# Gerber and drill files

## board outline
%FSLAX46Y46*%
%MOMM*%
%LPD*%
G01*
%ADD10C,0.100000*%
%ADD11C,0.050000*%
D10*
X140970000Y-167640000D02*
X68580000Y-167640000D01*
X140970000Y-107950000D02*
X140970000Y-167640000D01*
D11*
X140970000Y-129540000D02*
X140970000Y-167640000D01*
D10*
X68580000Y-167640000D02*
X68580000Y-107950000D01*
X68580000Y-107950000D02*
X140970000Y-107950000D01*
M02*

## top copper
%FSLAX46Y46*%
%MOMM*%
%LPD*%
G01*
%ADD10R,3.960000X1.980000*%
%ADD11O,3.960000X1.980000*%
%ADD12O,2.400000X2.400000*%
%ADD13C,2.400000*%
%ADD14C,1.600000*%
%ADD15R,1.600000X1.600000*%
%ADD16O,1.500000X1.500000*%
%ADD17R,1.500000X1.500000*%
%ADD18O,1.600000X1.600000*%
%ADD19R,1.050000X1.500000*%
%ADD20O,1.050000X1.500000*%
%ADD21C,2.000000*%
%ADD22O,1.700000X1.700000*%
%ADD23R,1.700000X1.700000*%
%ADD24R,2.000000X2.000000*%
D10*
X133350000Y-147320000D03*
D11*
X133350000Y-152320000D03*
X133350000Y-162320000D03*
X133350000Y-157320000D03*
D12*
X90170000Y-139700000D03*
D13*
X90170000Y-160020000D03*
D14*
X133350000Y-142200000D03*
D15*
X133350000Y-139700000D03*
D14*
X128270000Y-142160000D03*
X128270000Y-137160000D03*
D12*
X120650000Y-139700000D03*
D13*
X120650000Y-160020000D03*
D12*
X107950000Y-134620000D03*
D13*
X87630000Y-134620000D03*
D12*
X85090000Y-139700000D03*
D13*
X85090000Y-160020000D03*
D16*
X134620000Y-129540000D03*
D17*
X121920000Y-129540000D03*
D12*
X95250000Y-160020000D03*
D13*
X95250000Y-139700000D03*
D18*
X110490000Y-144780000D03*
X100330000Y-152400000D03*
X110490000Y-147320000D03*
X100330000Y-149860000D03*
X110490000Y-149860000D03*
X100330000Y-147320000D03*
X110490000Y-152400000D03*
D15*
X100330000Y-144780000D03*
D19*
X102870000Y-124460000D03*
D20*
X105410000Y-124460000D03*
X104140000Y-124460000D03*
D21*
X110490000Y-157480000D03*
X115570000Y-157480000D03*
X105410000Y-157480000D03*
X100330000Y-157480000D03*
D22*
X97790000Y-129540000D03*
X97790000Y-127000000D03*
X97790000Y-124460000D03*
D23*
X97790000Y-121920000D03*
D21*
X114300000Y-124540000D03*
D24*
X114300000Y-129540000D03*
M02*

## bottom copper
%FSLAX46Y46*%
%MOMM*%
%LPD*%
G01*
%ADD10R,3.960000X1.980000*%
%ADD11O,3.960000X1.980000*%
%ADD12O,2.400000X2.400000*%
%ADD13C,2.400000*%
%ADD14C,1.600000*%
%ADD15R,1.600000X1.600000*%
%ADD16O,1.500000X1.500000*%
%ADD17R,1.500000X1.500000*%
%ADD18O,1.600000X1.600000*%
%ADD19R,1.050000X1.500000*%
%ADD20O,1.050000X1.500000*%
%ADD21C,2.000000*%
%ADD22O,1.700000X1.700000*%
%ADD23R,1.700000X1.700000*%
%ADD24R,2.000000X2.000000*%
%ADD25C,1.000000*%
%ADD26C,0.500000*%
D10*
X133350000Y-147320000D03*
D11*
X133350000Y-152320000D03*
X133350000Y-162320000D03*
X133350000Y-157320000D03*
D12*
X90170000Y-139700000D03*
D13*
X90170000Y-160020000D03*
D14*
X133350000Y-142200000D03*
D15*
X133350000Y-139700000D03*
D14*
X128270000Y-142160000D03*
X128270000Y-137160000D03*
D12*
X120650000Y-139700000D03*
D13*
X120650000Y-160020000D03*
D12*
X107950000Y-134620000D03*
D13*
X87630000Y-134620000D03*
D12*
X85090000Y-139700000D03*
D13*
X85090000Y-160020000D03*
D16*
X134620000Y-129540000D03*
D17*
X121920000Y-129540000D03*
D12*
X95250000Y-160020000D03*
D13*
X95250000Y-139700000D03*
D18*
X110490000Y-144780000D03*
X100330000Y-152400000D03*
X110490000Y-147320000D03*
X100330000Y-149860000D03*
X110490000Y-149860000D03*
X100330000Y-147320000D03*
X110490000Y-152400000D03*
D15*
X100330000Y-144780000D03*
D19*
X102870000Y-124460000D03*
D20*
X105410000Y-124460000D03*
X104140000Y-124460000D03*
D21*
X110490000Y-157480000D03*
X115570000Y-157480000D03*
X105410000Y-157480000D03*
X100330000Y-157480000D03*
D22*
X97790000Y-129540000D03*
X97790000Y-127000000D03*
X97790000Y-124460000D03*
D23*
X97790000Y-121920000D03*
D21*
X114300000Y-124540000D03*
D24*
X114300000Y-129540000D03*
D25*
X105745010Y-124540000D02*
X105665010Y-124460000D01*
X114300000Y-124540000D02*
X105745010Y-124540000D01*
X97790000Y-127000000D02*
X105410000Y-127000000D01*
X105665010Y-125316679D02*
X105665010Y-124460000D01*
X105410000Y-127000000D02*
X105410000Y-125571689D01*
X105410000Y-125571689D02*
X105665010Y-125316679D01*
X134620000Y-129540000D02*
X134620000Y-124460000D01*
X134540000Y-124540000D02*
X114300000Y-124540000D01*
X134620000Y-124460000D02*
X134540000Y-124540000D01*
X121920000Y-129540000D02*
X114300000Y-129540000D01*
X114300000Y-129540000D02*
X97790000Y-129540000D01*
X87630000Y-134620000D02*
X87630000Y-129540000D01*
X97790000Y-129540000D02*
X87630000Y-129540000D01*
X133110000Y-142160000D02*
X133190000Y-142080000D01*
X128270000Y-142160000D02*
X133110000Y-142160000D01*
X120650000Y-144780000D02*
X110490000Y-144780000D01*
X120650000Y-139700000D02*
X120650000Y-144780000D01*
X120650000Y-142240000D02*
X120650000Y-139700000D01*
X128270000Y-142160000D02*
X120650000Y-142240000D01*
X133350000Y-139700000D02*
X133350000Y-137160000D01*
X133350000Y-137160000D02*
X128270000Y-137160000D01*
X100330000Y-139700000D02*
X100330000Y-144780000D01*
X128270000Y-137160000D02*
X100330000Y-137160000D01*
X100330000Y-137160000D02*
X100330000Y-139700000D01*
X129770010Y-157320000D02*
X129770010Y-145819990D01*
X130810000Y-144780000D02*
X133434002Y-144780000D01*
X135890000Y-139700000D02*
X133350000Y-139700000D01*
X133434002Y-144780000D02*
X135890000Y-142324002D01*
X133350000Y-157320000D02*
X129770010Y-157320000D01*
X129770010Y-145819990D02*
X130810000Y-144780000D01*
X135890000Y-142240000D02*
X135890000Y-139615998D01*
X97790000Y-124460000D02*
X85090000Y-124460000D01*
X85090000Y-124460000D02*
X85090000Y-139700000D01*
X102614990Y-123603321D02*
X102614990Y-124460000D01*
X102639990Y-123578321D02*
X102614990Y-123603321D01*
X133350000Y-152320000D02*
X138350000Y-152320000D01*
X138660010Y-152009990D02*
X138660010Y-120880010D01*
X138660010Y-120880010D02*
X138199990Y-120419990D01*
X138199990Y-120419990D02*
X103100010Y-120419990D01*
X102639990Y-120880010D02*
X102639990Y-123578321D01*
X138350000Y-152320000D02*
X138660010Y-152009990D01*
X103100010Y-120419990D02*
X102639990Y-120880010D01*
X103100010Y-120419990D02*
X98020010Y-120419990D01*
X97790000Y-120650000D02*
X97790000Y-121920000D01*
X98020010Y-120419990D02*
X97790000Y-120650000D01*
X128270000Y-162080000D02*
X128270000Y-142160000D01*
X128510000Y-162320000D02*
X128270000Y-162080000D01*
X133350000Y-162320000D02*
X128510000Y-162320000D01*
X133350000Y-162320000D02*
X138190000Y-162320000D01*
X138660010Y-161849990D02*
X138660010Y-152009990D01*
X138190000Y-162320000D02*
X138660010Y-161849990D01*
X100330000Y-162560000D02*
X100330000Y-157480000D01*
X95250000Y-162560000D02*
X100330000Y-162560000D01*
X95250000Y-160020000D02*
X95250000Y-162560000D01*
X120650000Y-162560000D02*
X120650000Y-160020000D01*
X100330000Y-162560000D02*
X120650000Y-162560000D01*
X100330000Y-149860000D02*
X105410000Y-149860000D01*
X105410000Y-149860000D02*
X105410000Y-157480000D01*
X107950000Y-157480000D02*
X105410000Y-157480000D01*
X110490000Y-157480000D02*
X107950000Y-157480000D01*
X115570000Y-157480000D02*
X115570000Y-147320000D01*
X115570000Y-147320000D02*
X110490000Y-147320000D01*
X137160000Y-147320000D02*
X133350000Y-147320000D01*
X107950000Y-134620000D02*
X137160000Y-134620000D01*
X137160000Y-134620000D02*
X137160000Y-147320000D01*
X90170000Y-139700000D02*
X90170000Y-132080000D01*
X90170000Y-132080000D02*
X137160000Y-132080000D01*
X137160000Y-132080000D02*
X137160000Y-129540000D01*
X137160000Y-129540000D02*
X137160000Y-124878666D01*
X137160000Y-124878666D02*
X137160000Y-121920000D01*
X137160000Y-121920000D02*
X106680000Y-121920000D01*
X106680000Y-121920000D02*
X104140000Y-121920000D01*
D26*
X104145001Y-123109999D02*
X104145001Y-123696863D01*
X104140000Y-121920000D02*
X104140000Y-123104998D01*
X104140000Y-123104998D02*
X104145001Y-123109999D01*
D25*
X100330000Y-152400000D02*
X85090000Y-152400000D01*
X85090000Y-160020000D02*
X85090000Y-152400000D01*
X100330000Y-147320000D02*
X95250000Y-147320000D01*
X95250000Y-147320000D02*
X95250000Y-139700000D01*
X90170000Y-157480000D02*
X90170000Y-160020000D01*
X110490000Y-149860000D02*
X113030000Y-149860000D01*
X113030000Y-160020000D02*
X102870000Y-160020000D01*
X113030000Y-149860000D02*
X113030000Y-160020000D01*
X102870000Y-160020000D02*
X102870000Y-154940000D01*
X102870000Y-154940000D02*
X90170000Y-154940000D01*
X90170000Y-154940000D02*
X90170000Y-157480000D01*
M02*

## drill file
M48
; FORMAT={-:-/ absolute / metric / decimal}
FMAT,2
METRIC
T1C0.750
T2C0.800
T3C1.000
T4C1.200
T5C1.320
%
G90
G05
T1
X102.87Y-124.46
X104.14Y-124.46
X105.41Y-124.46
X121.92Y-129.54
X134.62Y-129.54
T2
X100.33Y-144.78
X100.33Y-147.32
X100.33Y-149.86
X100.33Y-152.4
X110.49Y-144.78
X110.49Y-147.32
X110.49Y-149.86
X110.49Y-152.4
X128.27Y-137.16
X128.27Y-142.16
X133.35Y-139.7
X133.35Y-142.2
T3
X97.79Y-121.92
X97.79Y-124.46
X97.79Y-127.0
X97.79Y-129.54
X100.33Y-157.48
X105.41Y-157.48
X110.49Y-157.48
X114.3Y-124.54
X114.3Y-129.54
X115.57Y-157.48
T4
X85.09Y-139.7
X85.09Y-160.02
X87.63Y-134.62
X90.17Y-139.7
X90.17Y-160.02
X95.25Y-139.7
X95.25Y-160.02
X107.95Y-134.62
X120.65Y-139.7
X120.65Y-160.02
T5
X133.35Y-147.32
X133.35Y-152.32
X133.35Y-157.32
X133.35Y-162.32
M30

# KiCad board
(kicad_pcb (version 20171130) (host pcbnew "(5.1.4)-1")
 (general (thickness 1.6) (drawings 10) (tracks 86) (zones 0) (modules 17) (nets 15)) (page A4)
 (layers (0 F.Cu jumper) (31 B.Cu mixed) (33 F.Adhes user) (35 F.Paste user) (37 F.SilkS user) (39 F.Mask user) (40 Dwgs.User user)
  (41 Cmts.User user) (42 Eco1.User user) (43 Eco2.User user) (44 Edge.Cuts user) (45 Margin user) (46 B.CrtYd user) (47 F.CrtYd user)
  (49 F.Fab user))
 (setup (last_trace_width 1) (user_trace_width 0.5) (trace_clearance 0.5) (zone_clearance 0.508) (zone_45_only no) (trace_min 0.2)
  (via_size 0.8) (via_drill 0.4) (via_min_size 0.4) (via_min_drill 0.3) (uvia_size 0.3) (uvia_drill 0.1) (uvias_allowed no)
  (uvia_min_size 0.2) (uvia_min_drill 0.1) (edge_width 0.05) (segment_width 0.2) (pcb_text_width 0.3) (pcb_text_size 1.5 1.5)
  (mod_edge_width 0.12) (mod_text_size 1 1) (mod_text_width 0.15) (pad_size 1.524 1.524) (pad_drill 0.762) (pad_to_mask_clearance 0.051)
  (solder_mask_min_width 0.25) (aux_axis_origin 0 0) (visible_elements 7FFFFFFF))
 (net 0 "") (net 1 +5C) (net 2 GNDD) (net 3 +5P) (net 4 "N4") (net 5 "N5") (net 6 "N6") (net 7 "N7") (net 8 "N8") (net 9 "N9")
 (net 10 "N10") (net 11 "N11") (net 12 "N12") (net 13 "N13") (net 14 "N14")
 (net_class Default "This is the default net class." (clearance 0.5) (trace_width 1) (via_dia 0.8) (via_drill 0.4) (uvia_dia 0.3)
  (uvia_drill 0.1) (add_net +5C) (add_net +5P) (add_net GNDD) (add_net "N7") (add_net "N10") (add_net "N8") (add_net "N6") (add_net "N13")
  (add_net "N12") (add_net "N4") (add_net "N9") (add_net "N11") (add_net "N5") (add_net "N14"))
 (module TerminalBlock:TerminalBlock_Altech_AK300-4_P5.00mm (layer F.Cu) (at 133.35 147.32 270)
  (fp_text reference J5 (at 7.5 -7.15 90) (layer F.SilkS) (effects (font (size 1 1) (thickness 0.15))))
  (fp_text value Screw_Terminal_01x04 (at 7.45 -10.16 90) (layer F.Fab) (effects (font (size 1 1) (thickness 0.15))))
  (pad 1 thru_hole rect (at 0 0 270) (size 1.98 3.96) (drill 1.32) (layers *.Cu *.Mask) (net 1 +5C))
  (pad 2 thru_hole oval (at 5 0 270) (size 1.98 3.96) (drill 1.32) (layers *.Cu *.Mask) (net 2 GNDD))
  (pad 4 thru_hole oval (at 15 0 270) (size 1.98 3.96) (drill 1.32) (layers *.Cu *.Mask) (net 2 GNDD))
  (pad 3 thru_hole oval (at 10 0 270) (size 1.98 3.96) (drill 1.32) (layers *.Cu *.Mask) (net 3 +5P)))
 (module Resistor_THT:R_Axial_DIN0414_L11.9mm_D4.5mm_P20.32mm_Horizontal (layer F.Cu) (at 90.17 160.02 90)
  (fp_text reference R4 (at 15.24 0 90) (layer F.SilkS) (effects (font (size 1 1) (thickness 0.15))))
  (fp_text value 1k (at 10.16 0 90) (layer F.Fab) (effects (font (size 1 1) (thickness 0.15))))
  (pad 2 thru_hole oval (at 20.32 0 90) (size 2.4 2.4) (drill 1.2) (layers *.Cu *.Mask) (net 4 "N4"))
  (pad 1 thru_hole circle (at 0 0 90) (size 2.4 2.4) (drill 1.2) (layers *.Cu *.Mask) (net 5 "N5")))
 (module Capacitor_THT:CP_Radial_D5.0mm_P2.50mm (layer F.Cu) (at 133.35 139.7 270)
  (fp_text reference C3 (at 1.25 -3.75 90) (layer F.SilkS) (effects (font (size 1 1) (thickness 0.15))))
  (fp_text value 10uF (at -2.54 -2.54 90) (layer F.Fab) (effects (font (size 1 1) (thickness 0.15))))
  (pad 2 thru_hole circle (at 2.5 0 270) (size 1.6 1.6) (drill 0.8) (layers *.Cu *.Mask) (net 2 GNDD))
  (pad 1 thru_hole rect (at 0 0 270) (size 1.6 1.6) (drill 0.8) (layers *.Cu *.Mask) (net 3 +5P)))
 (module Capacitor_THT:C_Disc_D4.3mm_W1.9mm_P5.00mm (layer F.Cu) (at 128.27 137.16 270)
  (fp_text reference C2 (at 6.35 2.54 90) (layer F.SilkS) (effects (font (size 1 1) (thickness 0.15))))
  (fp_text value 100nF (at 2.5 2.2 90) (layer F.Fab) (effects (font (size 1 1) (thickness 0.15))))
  (pad 2 thru_hole circle (at 5 0 270) (size 1.6 1.6) (drill 0.8) (layers *.Cu *.Mask) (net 2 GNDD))
  (pad 1 thru_hole circle (at 0 0 270) (size 1.6 1.6) (drill 0.8) (layers *.Cu *.Mask) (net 3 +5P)))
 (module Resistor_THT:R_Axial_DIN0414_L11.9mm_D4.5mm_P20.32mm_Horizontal (layer F.Cu) (at 120.65 160.02 90)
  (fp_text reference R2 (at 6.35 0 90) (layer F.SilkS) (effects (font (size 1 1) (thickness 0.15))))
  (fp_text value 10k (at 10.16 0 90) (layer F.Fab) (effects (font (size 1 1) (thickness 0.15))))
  (pad 2 thru_hole oval (at 20.32 0 90) (size 2.4 2.4) (drill 1.2) (layers *.Cu *.Mask) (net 2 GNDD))
  (pad 1 thru_hole circle (at 0 0 90) (size 2.4 2.4) (drill 1.2) (layers *.Cu *.Mask) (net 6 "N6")))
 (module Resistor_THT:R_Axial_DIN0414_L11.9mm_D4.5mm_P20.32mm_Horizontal (layer F.Cu) (at 87.63 134.62)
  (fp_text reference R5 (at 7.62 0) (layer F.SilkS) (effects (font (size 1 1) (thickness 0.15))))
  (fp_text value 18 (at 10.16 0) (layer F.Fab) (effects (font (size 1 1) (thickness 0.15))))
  (pad 2 thru_hole oval (at 20.32 0) (size 2.4 2.4) (drill 1.2) (layers *.Cu *.Mask) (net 1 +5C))
  (pad 1 thru_hole circle (at 0 0) (size 2.4 2.4) (drill 1.2) (layers *.Cu *.Mask) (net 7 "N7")))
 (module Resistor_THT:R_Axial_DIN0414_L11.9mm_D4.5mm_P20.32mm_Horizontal (layer F.Cu) (at 85.09 160.02 90)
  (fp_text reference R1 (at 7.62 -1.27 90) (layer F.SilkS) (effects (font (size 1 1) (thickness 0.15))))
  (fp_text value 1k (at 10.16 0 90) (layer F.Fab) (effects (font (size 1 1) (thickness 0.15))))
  (pad 2 thru_hole oval (at 20.32 0 90) (size 2.4 2.4) (drill 1.2) (layers *.Cu *.Mask) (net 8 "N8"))
  (pad 1 thru_hole circle (at 0 0 90) (size 2.4 2.4) (drill 1.2) (layers *.Cu *.Mask) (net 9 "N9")))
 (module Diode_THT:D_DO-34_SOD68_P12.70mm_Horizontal (layer F.Cu) (at 121.92 129.54)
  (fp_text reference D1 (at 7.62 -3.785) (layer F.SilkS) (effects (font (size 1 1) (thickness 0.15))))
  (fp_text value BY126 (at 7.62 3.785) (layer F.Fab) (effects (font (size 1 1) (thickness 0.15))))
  (pad 2 thru_hole oval (at 12.7 0) (size 1.5 1.5) (drill 0.75) (layers *.Cu *.Mask) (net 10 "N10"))
  (pad 1 thru_hole rect (at 0 0) (size 1.5 1.5) (drill 0.75) (layers *.Cu *.Mask) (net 7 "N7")))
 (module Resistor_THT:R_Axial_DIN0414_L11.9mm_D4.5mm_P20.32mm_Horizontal (layer F.Cu) (at 95.25 139.7 270)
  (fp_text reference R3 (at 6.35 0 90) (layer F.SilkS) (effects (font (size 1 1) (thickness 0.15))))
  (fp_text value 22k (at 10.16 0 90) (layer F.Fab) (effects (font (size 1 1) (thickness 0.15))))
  (pad 2 thru_hole oval (at 20.32 0 270) (size 2.4 2.4) (drill 1.2) (layers *.Cu *.Mask) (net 6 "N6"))
  (pad 1 thru_hole circle (at 0 0 270) (size 2.4 2.4) (drill 1.2) (layers *.Cu *.Mask) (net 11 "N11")))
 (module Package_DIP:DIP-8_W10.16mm (layer F.Cu) (at 100.33 144.78)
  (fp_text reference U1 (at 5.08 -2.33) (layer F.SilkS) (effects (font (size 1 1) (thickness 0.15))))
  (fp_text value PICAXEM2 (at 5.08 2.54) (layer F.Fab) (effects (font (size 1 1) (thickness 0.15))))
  (pad 8 thru_hole oval (at 10.16 0) (size 1.6 1.6) (drill 0.8) (layers *.Cu *.Mask) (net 2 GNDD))
  (pad 4 thru_hole oval (at 0 7.62) (size 1.6 1.6) (drill 0.8) (layers *.Cu *.Mask) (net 9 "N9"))
  (pad 7 thru_hole oval (at 10.16 2.54) (size 1.6 1.6) (drill 0.8) (layers *.Cu *.Mask) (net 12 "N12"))
  (pad 3 thru_hole oval (at 0 5.08) (size 1.6 1.6) (drill 0.8) (layers *.Cu *.Mask) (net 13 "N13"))
  (pad 6 thru_hole oval (at 10.16 5.08) (size 1.6 1.6) (drill 0.8) (layers *.Cu *.Mask) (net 5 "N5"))
  (pad 2 thru_hole oval (at 0 2.54) (size 1.6 1.6) (drill 0.8) (layers *.Cu *.Mask) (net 11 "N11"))
  (pad 5 thru_hole oval (at 10.16 7.62) (size 1.6 1.6) (drill 0.8) (layers *.Cu *.Mask) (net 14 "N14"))
  (pad 1 thru_hole rect (at 0 0) (size 1.6 1.6) (drill 0.8) (layers *.Cu *.Mask) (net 3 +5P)))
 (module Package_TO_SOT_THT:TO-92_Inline (layer F.Cu) (at 102.87 124.46)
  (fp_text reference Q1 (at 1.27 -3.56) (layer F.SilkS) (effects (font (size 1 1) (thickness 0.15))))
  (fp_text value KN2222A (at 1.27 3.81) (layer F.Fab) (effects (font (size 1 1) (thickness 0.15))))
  (pad 1 thru_hole rect (at 0 0) (size 1.05 1.5) (drill 0.75) (layers *.Cu *.Mask) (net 2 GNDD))
  (pad 3 thru_hole oval (at 2.54 0) (size 1.05 1.5) (drill 0.75) (layers *.Cu *.Mask) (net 10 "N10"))
  (pad 2 thru_hole oval (at 1.27 0) (size 1.05 1.5) (drill 0.75) (layers *.Cu *.Mask) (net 4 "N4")))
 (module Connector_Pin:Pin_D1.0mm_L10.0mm (layer F.Cu) (at 110.49 157.48)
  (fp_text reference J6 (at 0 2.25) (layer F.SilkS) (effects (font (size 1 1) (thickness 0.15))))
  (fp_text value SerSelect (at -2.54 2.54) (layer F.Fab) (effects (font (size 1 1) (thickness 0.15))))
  (pad 1 thru_hole circle (at 0 0) (size 2 2) (drill 1) (layers *.Cu *.Mask) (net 13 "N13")))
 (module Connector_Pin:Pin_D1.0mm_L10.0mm (layer F.Cu) (at 115.57 157.48)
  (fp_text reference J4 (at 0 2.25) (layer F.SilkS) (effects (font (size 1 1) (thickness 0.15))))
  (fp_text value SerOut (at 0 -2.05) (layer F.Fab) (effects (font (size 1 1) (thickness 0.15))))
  (pad 1 thru_hole circle (at 0 0) (size 2 2) (drill 1) (layers *.Cu *.Mask) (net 12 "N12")))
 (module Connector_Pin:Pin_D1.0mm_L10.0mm (layer F.Cu) (at 105.41 157.48)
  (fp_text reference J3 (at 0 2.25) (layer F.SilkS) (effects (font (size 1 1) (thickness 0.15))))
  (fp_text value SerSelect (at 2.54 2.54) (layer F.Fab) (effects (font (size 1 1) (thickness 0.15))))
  (pad 1 thru_hole circle (at 0 0) (size 2 2) (drill 1) (layers *.Cu *.Mask) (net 13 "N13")))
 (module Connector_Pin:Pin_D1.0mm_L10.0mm (layer F.Cu) (at 100.33 157.48)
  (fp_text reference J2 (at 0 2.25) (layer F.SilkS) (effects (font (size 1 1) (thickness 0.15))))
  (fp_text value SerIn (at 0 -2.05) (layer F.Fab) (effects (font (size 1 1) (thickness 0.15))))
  (pad 1 thru_hole circle (at 0 0) (size 2 2) (drill 1) (layers *.Cu *.Mask) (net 6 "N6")))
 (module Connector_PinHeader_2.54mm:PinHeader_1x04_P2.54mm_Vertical (layer F.Cu) (at 97.79 121.92)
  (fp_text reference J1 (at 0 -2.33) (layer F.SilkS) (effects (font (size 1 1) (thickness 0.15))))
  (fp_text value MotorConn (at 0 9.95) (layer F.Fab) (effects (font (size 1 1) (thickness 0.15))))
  (pad 4 thru_hole oval (at 0 7.62) (size 1.7 1.7) (drill 1) (layers *.Cu *.Mask) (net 7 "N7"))
  (pad 3 thru_hole oval (at 0 5.08) (size 1.7 1.7) (drill 1) (layers *.Cu *.Mask) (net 10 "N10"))
  (pad 2 thru_hole oval (at 0 2.54) (size 1.7 1.7) (drill 1) (layers *.Cu *.Mask) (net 8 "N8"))
  (pad 1 thru_hole rect (at 0 0) (size 1.7 1.7) (drill 1) (layers *.Cu *.Mask) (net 2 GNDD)))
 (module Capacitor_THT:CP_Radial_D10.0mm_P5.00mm (layer F.Cu) (at 114.3 129.54 90)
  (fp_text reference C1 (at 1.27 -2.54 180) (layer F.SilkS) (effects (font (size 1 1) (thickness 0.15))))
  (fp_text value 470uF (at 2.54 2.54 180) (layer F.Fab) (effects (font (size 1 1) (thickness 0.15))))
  (pad 2 thru_hole circle (at 5 0 90) (size 2 2) (drill 1) (layers *.Cu *.Mask) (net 10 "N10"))
  (pad 1 thru_hole rect (at 0 0 90) (size 2 2) (drill 1) (layers *.Cu *.Mask) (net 7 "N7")))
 (gr_line (start 140.97 167.64) (end 68.58 167.64) (layer Edge.Cuts) (width 0.1))
 (gr_line (start 140.97 107.95) (end 140.97 167.64) (layer Edge.Cuts) (width 0.1))
 (gr_line (start 140.97 129.54) (end 140.97 167.64) (layer Edge.Cuts) (width 0.05))
 (gr_line (start 68.58 167.64) (end 68.58 107.95) (layer Edge.Cuts) (width 0.1))
 (gr_line (start 68.58 107.95) (end 140.97 107.95) (layer Edge.Cuts) (width 0.1))
 (segment (start 105.74501 124.54) (end 105.66501 124.46) (width 1) (layer B.Cu) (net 10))
 (segment (start 114.3 124.54) (end 105.74501 124.54) (width 1) (layer B.Cu) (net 10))
 (segment (start 97.79 127) (end 105.41 127) (width 1) (layer B.Cu) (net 10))
 (segment (start 105.66501 125.316679) (end 105.66501 124.46) (width 1) (layer B.Cu) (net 10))
 (segment (start 105.41 127) (end 105.41 125.571689) (width 1) (layer B.Cu) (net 10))
 (segment (start 105.41 125.571689) (end 105.66501 125.316679) (width 1) (layer B.Cu) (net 10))
 (segment (start 134.62 129.54) (end 134.62 124.46) (width 1) (layer B.Cu) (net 10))
 (segment (start 134.54 124.54) (end 114.3 124.54) (width 1) (layer B.Cu) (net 10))
 (segment (start 134.62 124.46) (end 134.54 124.54) (width 1) (layer B.Cu) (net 10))
 (segment (start 121.92 129.54) (end 114.3 129.54) (width 1) (layer B.Cu) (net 7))
 (segment (start 114.3 129.54) (end 97.79 129.54) (width 1) (layer B.Cu) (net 7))
 (segment (start 87.63 134.62) (end 87.63 129.54) (width 1) (layer B.Cu) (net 7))
 (segment (start 97.79 129.54) (end 87.63 129.54) (width 1) (layer B.Cu) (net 7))
 (segment (start 133.11 142.16) (end 133.19 142.08) (width 1) (layer B.Cu) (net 2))
 (segment (start 128.27 142.16) (end 133.11 142.16) (width 1) (layer B.Cu) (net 2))
 (segment (start 120.65 144.78) (end 110.49 144.78) (width 1) (layer B.Cu) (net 2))
 (segment (start 120.65 139.7) (end 120.65 144.78) (width 1) (layer B.Cu) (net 2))
 (segment (start 120.65 142.24) (end 120.65 139.7) (width 1) (layer B.Cu) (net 2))
 (segment (start 128.27 142.16) (end 120.65 142.24) (width 1) (layer B.Cu) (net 2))
 (segment (start 133.35 139.7) (end 133.35 137.16) (width 1) (layer B.Cu) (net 3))
 (segment (start 133.35 137.16) (end 128.27 137.16) (width 1) (layer B.Cu) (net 3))
 (segment (start 100.33 139.7) (end 100.33 144.78) (width 1) (layer B.Cu) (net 3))
 (segment (start 128.27 137.16) (end 100.33 137.16) (width 1) (layer B.Cu) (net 3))
 (segment (start 100.33 137.16) (end 100.33 139.7) (width 1) (layer B.Cu) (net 3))
 (segment (start 129.77001 157.32) (end 129.77001 145.81999) (width 1) (layer B.Cu) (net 3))
 (segment (start 130.81 144.78) (end 133.434002 144.78) (width 1) (layer B.Cu) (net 3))
 (segment (start 135.89 139.7) (end 133.35 139.7) (width 1) (layer B.Cu) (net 3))
 (segment (start 133.434002 144.78) (end 135.89 142.324002) (width 1) (layer B.Cu) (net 3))
 (segment (start 133.35 157.32) (end 129.77001 157.32) (width 1) (layer B.Cu) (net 3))
 (segment (start 129.77001 145.81999) (end 130.81 144.78) (width 1) (layer B.Cu) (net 3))
 (segment (start 135.89 142.24) (end 135.89 139.615998) (width 1) (layer B.Cu) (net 3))
 (segment (start 97.79 124.46) (end 85.09 124.46) (width 1) (layer B.Cu) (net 8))
 (segment (start 85.09 124.46) (end 85.09 139.7) (width 1) (layer B.Cu) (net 8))
 (segment (start 102.61499 123.603321) (end 102.61499 124.46) (width 1) (layer B.Cu) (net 2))
 (segment (start 102.63999 123.578321) (end 102.61499 123.603321) (width 1) (layer B.Cu) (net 2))
 (segment (start 133.35 152.32) (end 138.35 152.32) (width 1) (layer B.Cu) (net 2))
 (segment (start 138.66001 152.00999) (end 138.66001 120.88001) (width 1) (layer B.Cu) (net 2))
 (segment (start 138.66001 120.88001) (end 138.19999 120.41999) (width 1) (layer B.Cu) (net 2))
 (segment (start 138.19999 120.41999) (end 103.10001 120.41999) (width 1) (layer B.Cu) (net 2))
 (segment (start 102.63999 120.88001) (end 102.63999 123.578321) (width 1) (layer B.Cu) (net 2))
 (segment (start 138.35 152.32) (end 138.66001 152.00999) (width 1) (layer B.Cu) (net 2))
 (segment (start 103.10001 120.41999) (end 102.63999 120.88001) (width 1) (layer B.Cu) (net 2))
 (segment (start 103.10001 120.41999) (end 98.02001 120.41999) (width 1) (layer B.Cu) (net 2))
 (segment (start 97.79 120.65) (end 97.79 121.92) (width 1) (layer B.Cu) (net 2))
 (segment (start 98.02001 120.41999) (end 97.79 120.65) (width 1) (layer B.Cu) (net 2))
 (segment (start 128.27 162.08) (end 128.27 142.16) (width 1) (layer B.Cu) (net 2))
 (segment (start 128.51 162.32) (end 128.27 162.08) (width 1) (layer B.Cu) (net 2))
 (segment (start 133.35 162.32) (end 128.51 162.32) (width 1) (layer B.Cu) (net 2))
 (segment (start 133.35 162.32) (end 138.19 162.32) (width 1) (layer B.Cu) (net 2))
 (segment (start 138.66001 161.84999) (end 138.66001 152.00999) (width 1) (layer B.Cu) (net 2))
 (segment (start 138.19 162.32) (end 138.66001 161.84999) (width 1) (layer B.Cu) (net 2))
 (segment (start 100.33 162.56) (end 100.33 157.48) (width 1) (layer B.Cu) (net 6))
 (segment (start 95.25 162.56) (end 100.33 162.56) (width 1) (layer B.Cu) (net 6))
 (segment (start 95.25 160.02) (end 95.25 162.56) (width 1) (layer B.Cu) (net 6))
 (segment (start 120.65 162.56) (end 120.65 160.02) (width 1) (layer B.Cu) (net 6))
 (segment (start 100.33 162.56) (end 120.65 162.56) (width 1) (layer B.Cu) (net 6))
 (segment (start 100.33 149.86) (end 105.41 149.86) (width 1) (layer B.Cu) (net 13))
 (segment (start 105.41 149.86) (end 105.41 157.48) (width 1) (layer B.Cu) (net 13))
 (segment (start 107.95 157.48) (end 105.41 157.48) (width 1) (layer B.Cu) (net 13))
 (segment (start 110.49 157.48) (end 107.95 157.48) (width 1) (layer B.Cu) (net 13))
 (segment (start 115.57 157.48) (end 115.57 147.32) (width 1) (layer B.Cu) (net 12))
 (segment (start 115.57 147.32) (end 110.49 147.32) (width 1) (layer B.Cu) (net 12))
 (segment (start 137.16 147.32) (end 133.35 147.32) (width 1) (layer B.Cu) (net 1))
 (segment (start 107.95 134.62) (end 137.16 134.62) (width 1) (layer B.Cu) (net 1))
 (segment (start 137.16 134.62) (end 137.16 147.32) (width 1) (layer B.Cu) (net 1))
 (segment (start 90.17 139.7) (end 90.17 132.08) (width 1) (layer B.Cu) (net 4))
 (segment (start 90.17 132.08) (end 137.16 132.08) (width 1) (layer B.Cu) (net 4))
 (segment (start 137.16 132.08) (end 137.16 129.54) (width 1) (layer B.Cu) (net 4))
 (segment (start 137.16 129.54) (end 137.16 124.878666) (width 1) (layer B.Cu) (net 4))
 (segment (start 137.16 124.878666) (end 137.16 121.92) (width 1) (layer B.Cu) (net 4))
 (segment (start 137.16 121.92) (end 106.68 121.92) (width 1) (layer B.Cu) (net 4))
 (segment (start 106.68 121.92) (end 104.14 121.92) (width 1) (layer B.Cu) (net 4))
 (segment (start 104.145001 123.109999) (end 104.145001 123.696863) (width 0.5) (layer B.Cu) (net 4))
 (segment (start 104.14 121.92) (end 104.14 123.104998) (width 0.5) (layer B.Cu) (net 4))
 (segment (start 104.14 123.104998) (end 104.145001 123.109999) (width 0.5) (layer B.Cu) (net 4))
 (segment (start 100.33 152.4) (end 85.09 152.4) (width 1) (layer B.Cu) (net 9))
 (segment (start 85.09 160.02) (end 85.09 152.4) (width 1) (layer B.Cu) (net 9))
 (segment (start 100.33 147.32) (end 95.25 147.32) (width 1) (layer B.Cu) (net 11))
 (segment (start 95.25 147.32) (end 95.25 139.7) (width 1) (layer B.Cu) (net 11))
 (segment (start 90.17 157.48) (end 90.17 160.02) (width 1) (layer B.Cu) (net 5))
 (segment (start 110.49 149.86) (end 113.03 149.86) (width 1) (layer B.Cu) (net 5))
 (segment (start 113.03 160.02) (end 102.87 160.02) (width 1) (layer B.Cu) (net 5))
 (segment (start 113.03 149.86) (end 113.03 160.02) (width 1) (layer B.Cu) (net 5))
 (segment (start 102.87 160.02) (end 102.87 154.94) (width 1) (layer B.Cu) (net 5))
 (segment (start 102.87 154.94) (end 90.17 154.94) (width 1) (layer B.Cu) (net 5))
 (segment (start 90.17 154.94) (end 90.17 157.48) (width 1) (layer B.Cu) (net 5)))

